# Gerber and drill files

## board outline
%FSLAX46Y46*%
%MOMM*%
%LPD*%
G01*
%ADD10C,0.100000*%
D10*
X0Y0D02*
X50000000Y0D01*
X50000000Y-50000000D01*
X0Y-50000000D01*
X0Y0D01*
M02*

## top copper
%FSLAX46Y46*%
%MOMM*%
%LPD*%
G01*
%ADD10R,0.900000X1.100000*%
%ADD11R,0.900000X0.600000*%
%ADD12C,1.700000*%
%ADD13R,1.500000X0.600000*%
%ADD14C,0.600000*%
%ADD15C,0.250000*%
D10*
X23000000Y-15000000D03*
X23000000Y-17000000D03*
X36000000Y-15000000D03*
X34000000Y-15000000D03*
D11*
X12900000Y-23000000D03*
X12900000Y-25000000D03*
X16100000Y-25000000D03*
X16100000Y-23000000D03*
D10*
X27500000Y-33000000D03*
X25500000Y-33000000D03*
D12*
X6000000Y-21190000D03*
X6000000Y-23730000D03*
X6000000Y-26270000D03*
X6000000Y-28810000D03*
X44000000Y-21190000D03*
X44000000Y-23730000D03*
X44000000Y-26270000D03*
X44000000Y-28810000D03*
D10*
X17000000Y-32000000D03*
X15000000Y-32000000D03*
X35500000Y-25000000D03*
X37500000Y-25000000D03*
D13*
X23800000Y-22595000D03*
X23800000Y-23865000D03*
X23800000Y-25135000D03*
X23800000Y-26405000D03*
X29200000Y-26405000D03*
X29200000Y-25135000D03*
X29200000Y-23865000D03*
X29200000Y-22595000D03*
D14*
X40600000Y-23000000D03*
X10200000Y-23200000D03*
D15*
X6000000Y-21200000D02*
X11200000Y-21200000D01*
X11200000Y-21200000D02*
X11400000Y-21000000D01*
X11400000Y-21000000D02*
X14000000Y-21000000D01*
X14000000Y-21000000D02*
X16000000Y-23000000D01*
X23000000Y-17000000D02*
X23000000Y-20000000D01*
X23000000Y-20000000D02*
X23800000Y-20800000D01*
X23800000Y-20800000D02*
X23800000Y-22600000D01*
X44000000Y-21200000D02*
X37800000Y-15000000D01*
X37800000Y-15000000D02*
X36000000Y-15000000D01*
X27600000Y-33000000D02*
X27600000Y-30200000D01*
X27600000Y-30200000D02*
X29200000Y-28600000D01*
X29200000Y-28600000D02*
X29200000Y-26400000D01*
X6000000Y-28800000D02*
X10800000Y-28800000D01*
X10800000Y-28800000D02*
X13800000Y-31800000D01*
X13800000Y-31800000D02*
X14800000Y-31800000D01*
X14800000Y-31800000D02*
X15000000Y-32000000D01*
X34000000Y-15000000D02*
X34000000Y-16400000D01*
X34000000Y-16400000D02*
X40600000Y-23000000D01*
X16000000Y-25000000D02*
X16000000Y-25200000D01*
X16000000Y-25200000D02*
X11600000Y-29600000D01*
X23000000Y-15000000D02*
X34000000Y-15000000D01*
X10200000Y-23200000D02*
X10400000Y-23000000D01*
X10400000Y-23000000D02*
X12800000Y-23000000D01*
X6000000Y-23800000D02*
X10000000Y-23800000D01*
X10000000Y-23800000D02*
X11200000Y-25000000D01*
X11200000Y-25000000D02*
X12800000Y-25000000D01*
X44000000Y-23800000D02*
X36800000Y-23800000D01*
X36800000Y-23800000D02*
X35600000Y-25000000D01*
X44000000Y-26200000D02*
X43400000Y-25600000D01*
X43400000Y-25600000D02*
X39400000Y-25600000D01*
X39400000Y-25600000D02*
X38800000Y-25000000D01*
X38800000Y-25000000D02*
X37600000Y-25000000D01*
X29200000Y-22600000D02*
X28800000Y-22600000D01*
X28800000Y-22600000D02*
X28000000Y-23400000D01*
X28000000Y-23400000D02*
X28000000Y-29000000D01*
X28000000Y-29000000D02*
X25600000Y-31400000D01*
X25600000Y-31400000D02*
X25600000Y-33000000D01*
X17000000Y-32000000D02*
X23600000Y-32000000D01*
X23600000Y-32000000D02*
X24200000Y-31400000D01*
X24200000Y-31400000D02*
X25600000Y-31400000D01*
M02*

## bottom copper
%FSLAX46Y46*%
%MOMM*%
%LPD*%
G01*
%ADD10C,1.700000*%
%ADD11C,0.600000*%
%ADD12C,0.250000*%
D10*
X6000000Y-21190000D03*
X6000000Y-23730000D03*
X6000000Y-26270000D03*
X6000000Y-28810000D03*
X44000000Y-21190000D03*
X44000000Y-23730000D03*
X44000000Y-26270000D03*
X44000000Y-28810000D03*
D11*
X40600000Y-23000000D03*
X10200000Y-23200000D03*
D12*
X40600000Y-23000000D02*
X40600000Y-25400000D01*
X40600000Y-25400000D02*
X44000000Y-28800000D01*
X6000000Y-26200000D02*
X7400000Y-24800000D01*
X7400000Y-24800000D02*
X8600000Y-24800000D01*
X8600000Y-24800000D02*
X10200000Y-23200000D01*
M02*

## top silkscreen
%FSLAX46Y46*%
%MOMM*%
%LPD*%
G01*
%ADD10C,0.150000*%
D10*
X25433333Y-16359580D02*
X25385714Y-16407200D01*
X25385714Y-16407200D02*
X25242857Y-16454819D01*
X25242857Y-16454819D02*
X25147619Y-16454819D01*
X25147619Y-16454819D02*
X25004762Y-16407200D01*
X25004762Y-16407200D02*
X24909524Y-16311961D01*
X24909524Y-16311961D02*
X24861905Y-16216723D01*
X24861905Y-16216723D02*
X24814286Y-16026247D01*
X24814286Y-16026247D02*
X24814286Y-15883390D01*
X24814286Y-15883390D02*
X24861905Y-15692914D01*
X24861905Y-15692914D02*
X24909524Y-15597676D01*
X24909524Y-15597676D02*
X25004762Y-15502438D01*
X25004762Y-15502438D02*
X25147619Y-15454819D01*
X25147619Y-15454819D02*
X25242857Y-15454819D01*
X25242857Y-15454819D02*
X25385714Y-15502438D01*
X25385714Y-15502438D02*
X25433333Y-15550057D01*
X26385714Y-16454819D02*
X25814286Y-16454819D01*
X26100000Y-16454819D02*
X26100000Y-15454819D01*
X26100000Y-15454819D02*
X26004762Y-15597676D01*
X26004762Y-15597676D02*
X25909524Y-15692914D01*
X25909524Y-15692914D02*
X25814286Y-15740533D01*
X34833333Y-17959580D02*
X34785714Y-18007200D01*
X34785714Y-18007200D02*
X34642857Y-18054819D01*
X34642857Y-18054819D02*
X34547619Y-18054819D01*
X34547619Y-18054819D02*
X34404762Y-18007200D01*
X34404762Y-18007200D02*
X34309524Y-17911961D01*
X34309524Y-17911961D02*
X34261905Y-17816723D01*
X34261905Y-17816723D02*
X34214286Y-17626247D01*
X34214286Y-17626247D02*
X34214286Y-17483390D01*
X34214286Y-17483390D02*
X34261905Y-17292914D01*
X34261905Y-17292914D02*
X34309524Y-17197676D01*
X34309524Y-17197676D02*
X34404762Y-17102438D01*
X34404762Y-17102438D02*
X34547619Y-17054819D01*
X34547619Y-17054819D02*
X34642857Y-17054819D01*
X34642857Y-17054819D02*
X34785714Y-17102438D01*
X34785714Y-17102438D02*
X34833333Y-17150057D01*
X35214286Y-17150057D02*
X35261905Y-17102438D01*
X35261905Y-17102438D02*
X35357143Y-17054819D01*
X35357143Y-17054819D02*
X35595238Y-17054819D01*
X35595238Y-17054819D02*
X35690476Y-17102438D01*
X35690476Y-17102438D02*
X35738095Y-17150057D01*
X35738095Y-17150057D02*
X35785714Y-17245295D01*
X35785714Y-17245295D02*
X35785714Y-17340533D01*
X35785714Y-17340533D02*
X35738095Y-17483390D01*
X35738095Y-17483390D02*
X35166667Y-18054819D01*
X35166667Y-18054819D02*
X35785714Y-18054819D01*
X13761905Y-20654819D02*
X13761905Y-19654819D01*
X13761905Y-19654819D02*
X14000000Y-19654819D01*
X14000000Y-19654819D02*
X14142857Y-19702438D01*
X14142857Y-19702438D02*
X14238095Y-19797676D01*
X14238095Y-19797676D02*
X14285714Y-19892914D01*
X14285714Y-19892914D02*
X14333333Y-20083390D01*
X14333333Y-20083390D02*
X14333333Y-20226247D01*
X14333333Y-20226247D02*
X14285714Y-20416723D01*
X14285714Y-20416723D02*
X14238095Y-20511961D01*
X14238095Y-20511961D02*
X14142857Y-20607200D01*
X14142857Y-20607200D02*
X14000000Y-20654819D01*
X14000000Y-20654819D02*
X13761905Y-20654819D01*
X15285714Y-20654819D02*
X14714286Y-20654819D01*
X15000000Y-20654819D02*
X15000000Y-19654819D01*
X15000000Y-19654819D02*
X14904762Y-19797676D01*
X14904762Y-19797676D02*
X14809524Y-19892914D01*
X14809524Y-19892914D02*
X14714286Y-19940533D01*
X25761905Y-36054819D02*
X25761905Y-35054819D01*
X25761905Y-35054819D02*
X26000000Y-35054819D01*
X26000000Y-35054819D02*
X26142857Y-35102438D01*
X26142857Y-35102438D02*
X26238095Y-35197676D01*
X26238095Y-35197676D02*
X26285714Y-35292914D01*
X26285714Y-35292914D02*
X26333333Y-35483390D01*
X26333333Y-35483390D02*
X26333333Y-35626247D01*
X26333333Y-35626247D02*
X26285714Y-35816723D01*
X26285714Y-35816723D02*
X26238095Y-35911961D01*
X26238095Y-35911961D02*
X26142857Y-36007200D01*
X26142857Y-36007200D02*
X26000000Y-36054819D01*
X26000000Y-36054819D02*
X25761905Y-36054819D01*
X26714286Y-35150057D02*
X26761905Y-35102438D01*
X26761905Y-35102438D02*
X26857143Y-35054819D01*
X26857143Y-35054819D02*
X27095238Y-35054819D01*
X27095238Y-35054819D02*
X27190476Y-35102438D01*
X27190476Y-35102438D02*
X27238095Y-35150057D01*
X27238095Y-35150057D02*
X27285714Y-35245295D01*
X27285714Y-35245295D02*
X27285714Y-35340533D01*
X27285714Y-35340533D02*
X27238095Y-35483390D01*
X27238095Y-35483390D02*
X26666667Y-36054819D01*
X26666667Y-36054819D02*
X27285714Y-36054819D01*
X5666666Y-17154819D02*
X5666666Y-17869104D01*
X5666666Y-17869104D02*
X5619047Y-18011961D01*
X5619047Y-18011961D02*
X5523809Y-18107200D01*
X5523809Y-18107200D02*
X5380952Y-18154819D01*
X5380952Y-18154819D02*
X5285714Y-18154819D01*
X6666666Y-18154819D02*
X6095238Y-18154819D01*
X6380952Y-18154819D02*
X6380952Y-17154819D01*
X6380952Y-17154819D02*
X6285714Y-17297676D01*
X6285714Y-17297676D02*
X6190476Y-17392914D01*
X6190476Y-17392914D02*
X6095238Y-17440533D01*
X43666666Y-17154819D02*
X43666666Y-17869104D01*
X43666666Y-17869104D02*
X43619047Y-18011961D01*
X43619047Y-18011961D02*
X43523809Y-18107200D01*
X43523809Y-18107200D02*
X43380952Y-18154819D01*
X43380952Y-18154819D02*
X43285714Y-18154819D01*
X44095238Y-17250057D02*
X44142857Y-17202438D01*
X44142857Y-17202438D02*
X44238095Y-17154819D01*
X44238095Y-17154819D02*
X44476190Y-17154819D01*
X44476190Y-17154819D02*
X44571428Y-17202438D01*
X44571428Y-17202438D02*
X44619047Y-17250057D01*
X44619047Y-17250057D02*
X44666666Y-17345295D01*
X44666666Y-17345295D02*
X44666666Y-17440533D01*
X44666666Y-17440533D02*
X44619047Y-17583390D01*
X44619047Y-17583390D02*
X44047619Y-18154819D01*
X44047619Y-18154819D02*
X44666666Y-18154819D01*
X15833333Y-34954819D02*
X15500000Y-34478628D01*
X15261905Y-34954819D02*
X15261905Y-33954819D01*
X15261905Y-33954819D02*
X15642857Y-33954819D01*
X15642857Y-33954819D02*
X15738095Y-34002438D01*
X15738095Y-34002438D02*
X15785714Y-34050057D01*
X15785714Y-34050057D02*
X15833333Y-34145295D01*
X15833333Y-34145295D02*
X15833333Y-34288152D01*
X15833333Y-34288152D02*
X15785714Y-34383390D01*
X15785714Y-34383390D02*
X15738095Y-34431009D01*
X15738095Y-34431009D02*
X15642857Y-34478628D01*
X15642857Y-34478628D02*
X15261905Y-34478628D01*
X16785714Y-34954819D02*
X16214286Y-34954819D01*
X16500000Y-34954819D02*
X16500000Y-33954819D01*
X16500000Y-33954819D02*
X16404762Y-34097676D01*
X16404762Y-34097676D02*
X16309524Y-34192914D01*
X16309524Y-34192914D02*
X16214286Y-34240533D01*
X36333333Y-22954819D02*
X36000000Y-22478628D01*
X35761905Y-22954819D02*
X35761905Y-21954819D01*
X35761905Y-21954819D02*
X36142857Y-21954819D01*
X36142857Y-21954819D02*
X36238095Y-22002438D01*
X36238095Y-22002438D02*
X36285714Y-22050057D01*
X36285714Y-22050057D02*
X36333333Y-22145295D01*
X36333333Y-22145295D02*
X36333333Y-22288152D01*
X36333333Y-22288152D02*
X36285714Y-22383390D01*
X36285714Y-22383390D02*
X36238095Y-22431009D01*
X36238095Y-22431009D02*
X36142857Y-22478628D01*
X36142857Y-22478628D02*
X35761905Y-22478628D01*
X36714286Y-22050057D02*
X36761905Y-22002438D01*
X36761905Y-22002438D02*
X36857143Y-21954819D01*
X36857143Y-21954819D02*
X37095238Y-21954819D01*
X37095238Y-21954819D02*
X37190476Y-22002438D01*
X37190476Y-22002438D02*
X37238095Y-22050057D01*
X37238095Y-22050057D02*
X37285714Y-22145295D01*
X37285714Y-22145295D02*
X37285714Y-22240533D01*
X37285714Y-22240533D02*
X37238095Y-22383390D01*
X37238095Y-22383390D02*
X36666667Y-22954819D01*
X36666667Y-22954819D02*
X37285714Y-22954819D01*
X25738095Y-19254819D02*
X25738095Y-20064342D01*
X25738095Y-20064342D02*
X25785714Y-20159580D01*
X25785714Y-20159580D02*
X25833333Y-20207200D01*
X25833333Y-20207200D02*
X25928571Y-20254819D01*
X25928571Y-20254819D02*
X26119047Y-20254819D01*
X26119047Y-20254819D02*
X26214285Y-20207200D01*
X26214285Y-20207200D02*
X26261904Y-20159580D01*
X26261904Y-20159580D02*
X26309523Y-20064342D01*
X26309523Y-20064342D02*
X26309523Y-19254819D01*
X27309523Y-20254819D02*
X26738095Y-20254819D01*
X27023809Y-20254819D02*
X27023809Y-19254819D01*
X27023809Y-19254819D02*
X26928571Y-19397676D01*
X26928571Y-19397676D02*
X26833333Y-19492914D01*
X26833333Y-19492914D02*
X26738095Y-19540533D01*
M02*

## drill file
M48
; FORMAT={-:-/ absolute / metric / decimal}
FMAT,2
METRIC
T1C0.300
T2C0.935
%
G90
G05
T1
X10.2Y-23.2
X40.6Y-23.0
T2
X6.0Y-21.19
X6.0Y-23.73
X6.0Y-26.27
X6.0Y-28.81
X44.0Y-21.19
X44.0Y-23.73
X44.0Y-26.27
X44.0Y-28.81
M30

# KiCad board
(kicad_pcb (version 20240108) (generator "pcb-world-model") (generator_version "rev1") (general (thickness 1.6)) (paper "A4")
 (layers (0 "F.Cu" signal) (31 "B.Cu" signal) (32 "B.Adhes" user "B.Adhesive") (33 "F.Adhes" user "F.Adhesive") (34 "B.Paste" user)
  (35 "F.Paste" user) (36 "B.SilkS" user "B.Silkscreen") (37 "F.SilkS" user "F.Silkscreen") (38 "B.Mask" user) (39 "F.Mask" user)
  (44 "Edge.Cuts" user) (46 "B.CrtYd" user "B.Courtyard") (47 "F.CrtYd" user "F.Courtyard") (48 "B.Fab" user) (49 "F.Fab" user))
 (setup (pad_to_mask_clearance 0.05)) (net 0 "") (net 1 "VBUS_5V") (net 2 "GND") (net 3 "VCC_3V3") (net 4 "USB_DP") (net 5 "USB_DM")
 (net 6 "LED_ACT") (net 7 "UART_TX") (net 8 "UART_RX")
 (gr_rect (start 0.0 0.0) (end 50.0000 50.0000) (stroke (width 0.1) (type default)) (fill none) (layer "Edge.Cuts"))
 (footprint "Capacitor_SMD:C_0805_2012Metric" (layer "F.Cu") (at 23.0000 16.0000 270)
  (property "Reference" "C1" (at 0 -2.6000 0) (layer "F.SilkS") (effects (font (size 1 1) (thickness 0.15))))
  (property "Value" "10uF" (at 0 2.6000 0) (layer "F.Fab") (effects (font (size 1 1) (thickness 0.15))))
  (pad "1" smd rect (at -1.0000 0.0000) (size 0.9000 1.1000) (layers "F.Cu" "F.Paste" "F.Mask") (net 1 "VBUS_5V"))
  (pad "2" smd rect (at 1.0000 0.0000) (size 0.9000 1.1000) (layers "F.Cu" "F.Paste" "F.Mask") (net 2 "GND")))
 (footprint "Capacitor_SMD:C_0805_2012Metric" (layer "F.Cu") (at 35.0000 15.0000 180)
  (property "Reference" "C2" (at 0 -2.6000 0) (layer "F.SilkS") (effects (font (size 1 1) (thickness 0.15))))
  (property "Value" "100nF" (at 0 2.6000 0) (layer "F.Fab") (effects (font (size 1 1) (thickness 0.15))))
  (pad "1" smd rect (at -1.0000 0.0000) (size 0.9000 1.1000) (layers "F.Cu" "F.Paste" "F.Mask") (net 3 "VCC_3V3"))
  (pad "2" smd rect (at 1.0000 0.0000) (size 0.9000 1.1000) (layers "F.Cu" "F.Paste" "F.Mask") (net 2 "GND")))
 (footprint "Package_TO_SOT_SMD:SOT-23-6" (layer "F.Cu") (at 14.5000 24.0000 0)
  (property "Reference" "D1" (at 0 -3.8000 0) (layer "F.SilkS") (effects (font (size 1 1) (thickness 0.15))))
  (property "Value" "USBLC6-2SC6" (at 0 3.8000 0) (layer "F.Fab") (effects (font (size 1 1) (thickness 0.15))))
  (pad "1" smd rect (at -1.6000 -1.0000) (size 0.9000 0.6000) (layers "F.Cu" "F.Paste" "F.Mask") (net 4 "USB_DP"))
  (pad "2" smd rect (at -1.6000 1.0000) (size 0.9000 0.6000) (layers "F.Cu" "F.Paste" "F.Mask") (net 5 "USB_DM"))
  (pad "3" smd rect (at 1.6000 1.0000) (size 0.9000 0.6000) (layers "F.Cu" "F.Paste" "F.Mask") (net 2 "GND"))
  (pad "4" smd rect (at 1.6000 -1.0000) (size 0.9000 0.6000) (layers "F.Cu" "F.Paste" "F.Mask") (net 1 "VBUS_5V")))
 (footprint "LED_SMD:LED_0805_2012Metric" (layer "F.Cu") (at 26.5000 33.0000 180)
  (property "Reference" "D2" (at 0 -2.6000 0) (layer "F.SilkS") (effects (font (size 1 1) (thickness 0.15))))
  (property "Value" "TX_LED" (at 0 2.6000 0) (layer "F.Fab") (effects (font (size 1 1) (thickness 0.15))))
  (pad "1" smd rect (at -1.0000 0.0000) (size 0.9000 1.1000) (layers "F.Cu" "F.Paste" "F.Mask") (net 3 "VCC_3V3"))
  (pad "2" smd rect (at 1.0000 0.0000) (size 0.9000 1.1000) (layers "F.Cu" "F.Paste" "F.Mask") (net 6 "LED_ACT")))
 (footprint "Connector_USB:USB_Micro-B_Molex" (layer "F.Cu") (at 6.0000 25.0000 0) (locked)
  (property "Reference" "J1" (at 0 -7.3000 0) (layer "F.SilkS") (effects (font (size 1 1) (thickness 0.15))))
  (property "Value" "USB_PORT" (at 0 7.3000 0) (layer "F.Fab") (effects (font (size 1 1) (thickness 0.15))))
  (pad "1" thru_hole circle (at 0.0000 -3.8100) (size 1.7000 1.7000) (drill 0.9350) (layers "*.Cu" "*.Mask") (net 1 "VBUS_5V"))
  (pad "2" thru_hole circle (at 0.0000 -1.2700) (size 1.7000 1.7000) (drill 0.9350) (layers "*.Cu" "*.Mask") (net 5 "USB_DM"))
  (pad "3" thru_hole circle (at 0.0000 1.2700) (size 1.7000 1.7000) (drill 0.9350) (layers "*.Cu" "*.Mask") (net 4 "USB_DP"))
  (pad "4" thru_hole circle (at 0.0000 3.8100) (size 1.7000 1.7000) (drill 0.9350) (layers "*.Cu" "*.Mask") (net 2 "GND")))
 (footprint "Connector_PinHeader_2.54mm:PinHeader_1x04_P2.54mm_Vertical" (layer "F.Cu") (at 44.0000 25.0000 0) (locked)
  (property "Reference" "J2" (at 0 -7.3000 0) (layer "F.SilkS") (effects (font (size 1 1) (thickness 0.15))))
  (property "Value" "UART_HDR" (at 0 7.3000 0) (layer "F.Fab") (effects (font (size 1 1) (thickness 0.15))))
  (pad "1" thru_hole circle (at 0.0000 -3.8100) (size 1.7000 1.7000) (drill 0.9350) (layers "*.Cu" "*.Mask") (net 3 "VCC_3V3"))
  (pad "2" thru_hole circle (at 0.0000 -1.2700) (size 1.7000 1.7000) (drill 0.9350) (layers "*.Cu" "*.Mask") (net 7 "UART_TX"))
  (pad "3" thru_hole circle (at 0.0000 1.2700) (size 1.7000 1.7000) (drill 0.9350) (layers "*.Cu" "*.Mask") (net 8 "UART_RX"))
  (pad "4" thru_hole circle (at 0.0000 3.8100) (size 1.7000 1.7000) (drill 0.9350) (layers "*.Cu" "*.Mask") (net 2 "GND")))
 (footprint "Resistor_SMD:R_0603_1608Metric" (layer "F.Cu") (at 16.0000 32.0000 180)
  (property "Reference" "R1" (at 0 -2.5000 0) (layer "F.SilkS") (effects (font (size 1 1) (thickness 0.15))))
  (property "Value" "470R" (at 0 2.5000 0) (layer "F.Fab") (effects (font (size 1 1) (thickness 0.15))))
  (pad "1" smd rect (at -1.0000 0.0000) (size 0.9000 1.1000) (layers "F.Cu" "F.Paste" "F.Mask") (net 6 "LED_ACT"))
  (pad "2" smd rect (at 1.0000 0.0000) (size 0.9000 1.1000) (layers "F.Cu" "F.Paste" "F.Mask") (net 2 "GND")))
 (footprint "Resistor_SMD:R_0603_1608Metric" (layer "F.Cu") (at 36.5000 25.0000 0)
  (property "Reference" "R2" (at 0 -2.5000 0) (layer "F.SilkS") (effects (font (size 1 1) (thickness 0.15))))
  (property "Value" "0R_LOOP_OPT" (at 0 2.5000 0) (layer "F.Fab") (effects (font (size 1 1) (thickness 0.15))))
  (pad "1" smd rect (at -1.0000 0.0000) (size 0.9000 1.1000) (layers "F.Cu" "F.Paste" "F.Mask") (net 7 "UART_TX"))
  (pad "2" smd rect (at 1.0000 0.0000) (size 0.9000 1.1000) (layers "F.Cu" "F.Paste" "F.Mask") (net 8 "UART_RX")))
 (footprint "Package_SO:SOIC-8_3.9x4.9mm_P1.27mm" (layer "F.Cu") (at 26.5000 24.5000 0)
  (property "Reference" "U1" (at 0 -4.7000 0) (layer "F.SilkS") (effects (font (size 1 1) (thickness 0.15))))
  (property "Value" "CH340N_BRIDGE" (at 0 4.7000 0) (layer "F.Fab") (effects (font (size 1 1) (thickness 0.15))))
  (pad "1" smd rect (at -2.7000 -1.9050) (size 1.5000 0.6000) (layers "F.Cu" "F.Paste" "F.Mask") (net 1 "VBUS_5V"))
  (pad "2" smd rect (at -2.7000 -0.6350) (size 1.5000 0.6000) (layers "F.Cu" "F.Paste" "F.Mask") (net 4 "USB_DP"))
  (pad "3" smd rect (at -2.7000 0.6350) (size 1.5000 0.6000) (layers "F.Cu" "F.Paste" "F.Mask") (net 5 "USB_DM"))
  (pad "4" smd rect (at -2.7000 1.9050) (size 1.5000 0.6000) (layers "F.Cu" "F.Paste" "F.Mask") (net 2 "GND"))
  (pad "5" smd rect (at 2.7000 1.9050) (size 1.5000 0.6000) (layers "F.Cu" "F.Paste" "F.Mask") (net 3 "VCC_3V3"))
  (pad "6" smd rect (at 2.7000 0.6350) (size 1.5000 0.6000) (layers "F.Cu" "F.Paste" "F.Mask") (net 7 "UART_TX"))
  (pad "7" smd rect (at 2.7000 -0.6350) (size 1.5000 0.6000) (layers "F.Cu" "F.Paste" "F.Mask") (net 8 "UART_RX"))
  (pad "8" smd rect (at 2.7000 -1.9050) (size 1.5000 0.6000) (layers "F.Cu" "F.Paste" "F.Mask") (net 6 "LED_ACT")))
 (segment (start 6.0000 21.2000) (end 11.2000 21.2000) (width 0.2500) (layer "F.Cu") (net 1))
 (segment (start 11.2000 21.2000) (end 11.4000 21.0000) (width 0.2500) (layer "F.Cu") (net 1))
 (segment (start 11.4000 21.0000) (end 14.0000 21.0000) (width 0.2500) (layer "F.Cu") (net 1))
 (segment (start 14.0000 21.0000) (end 16.0000 23.0000) (width 0.2500) (layer "F.Cu") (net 1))
 (segment (start 23.0000 17.0000) (end 23.0000 20.0000) (width 0.2500) (layer "F.Cu") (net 1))
 (segment (start 23.0000 20.0000) (end 23.8000 20.8000) (width 0.2500) (layer "F.Cu") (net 1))
 (segment (start 23.8000 20.8000) (end 23.8000 22.6000) (width 0.2500) (layer "F.Cu") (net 1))
 (segment (start 44.0000 21.2000) (end 37.8000 15.0000) (width 0.2500) (layer "F.Cu") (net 3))
 (segment (start 37.8000 15.0000) (end 36.0000 15.0000) (width 0.2500) (layer "F.Cu") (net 3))
 (segment (start 27.6000 33.0000) (end 27.6000 30.2000) (width 0.2500) (layer "F.Cu") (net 3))
 (segment (start 27.6000 30.2000) (end 29.2000 28.6000) (width 0.2500) (layer "F.Cu") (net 3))
 (segment (start 29.2000 28.6000) (end 29.2000 26.4000) (width 0.2500) (layer "F.Cu") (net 3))
 (segment (start 6.0000 28.8000) (end 10.8000 28.8000) (width 0.2500) (layer "F.Cu") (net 2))
 (segment (start 10.8000 28.8000) (end 13.8000 31.8000) (width 0.2500) (layer "F.Cu") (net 2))
 (segment (start 13.8000 31.8000) (end 14.8000 31.8000) (width 0.2500) (layer "F.Cu") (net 2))
 (segment (start 14.8000 31.8000) (end 15.0000 32.0000) (width 0.2500) (layer "F.Cu") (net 2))
 (segment (start 34.0000 15.0000) (end 34.0000 16.4000) (width 0.2500) (layer "F.Cu") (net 2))
 (segment (start 34.0000 16.4000) (end 40.6000 23.0000) (width 0.2500) (layer "F.Cu") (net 2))
 (segment (start 40.6000 23.0000) (end 40.6000 25.4000) (width 0.2500) (layer "B.Cu") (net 2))
 (segment (start 40.6000 25.4000) (end 44.0000 28.8000) (width 0.2500) (layer "B.Cu") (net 2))
 (segment (start 16.0000 25.0000) (end 16.0000 25.2000) (width 0.2500) (layer "F.Cu") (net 2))
 (segment (start 16.0000 25.2000) (end 11.6000 29.6000) (width 0.2500) (layer "F.Cu") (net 2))
 (segment (start 23.0000 15.0000) (end 34.0000 15.0000) (width 0.2500) (layer "F.Cu") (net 2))
 (segment (start 6.0000 26.2000) (end 7.4000 24.8000) (width 0.2500) (layer "B.Cu") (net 4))
 (segment (start 7.4000 24.8000) (end 8.6000 24.8000) (width 0.2500) (layer "B.Cu") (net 4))
 (segment (start 8.6000 24.8000) (end 10.2000 23.2000) (width 0.2500) (layer "B.Cu") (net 4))
 (segment (start 10.2000 23.2000) (end 10.4000 23.0000) (width 0.2500) (layer "F.Cu") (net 4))
 (segment (start 10.4000 23.0000) (end 12.8000 23.0000) (width 0.2500) (layer "F.Cu") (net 4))
 (segment (start 6.0000 23.8000) (end 10.0000 23.8000) (width 0.2500) (layer "F.Cu") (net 5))
 (segment (start 10.0000 23.8000) (end 11.2000 25.0000) (width 0.2500) (layer "F.Cu") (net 5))
 (segment (start 11.2000 25.0000) (end 12.8000 25.0000) (width 0.2500) (layer "F.Cu") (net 5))
 (segment (start 44.0000 23.8000) (end 36.8000 23.8000) (width 0.2500) (layer "F.Cu") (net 7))
 (segment (start 36.8000 23.8000) (end 35.6000 25.0000) (width 0.2500) (layer "F.Cu") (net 7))
 (segment (start 44.0000 26.2000) (end 43.4000 25.6000) (width 0.2500) (layer "F.Cu") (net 8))
 (segment (start 43.4000 25.6000) (end 39.4000 25.6000) (width 0.2500) (layer "F.Cu") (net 8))
 (segment (start 39.4000 25.6000) (end 38.8000 25.0000) (width 0.2500) (layer "F.Cu") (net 8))
 (segment (start 38.8000 25.0000) (end 37.6000 25.0000) (width 0.2500) (layer "F.Cu") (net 8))
 (segment (start 29.2000 22.6000) (end 28.8000 22.6000) (width 0.2500) (layer "F.Cu") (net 6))
 (segment (start 28.8000 22.6000) (end 28.0000 23.4000) (width 0.2500) (layer "F.Cu") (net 6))
 (segment (start 28.0000 23.4000) (end 28.0000 29.0000) (width 0.2500) (layer "F.Cu") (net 6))
 (segment (start 28.0000 29.0000) (end 25.6000 31.4000) (width 0.2500) (layer "F.Cu") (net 6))
 (segment (start 25.6000 31.4000) (end 25.6000 33.0000) (width 0.2500) (layer "F.Cu") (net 6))
 (segment (start 17.0000 32.0000) (end 23.6000 32.0000) (width 0.2500) (layer "F.Cu") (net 6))
 (segment (start 23.6000 32.0000) (end 24.2000 31.4000) (width 0.2500) (layer "F.Cu") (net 6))
 (segment (start 24.2000 31.4000) (end 25.6000 31.4000) (width 0.2500) (layer "F.Cu") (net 6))
 (via (at 40.6000 23.0000) (size 0.6000) (drill 0.3000) (layers "F.Cu" "B.Cu") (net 2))
 (via (at 10.2000 23.2000) (size 0.6000) (drill 0.3000) (layers "F.Cu" "B.Cu") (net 4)))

